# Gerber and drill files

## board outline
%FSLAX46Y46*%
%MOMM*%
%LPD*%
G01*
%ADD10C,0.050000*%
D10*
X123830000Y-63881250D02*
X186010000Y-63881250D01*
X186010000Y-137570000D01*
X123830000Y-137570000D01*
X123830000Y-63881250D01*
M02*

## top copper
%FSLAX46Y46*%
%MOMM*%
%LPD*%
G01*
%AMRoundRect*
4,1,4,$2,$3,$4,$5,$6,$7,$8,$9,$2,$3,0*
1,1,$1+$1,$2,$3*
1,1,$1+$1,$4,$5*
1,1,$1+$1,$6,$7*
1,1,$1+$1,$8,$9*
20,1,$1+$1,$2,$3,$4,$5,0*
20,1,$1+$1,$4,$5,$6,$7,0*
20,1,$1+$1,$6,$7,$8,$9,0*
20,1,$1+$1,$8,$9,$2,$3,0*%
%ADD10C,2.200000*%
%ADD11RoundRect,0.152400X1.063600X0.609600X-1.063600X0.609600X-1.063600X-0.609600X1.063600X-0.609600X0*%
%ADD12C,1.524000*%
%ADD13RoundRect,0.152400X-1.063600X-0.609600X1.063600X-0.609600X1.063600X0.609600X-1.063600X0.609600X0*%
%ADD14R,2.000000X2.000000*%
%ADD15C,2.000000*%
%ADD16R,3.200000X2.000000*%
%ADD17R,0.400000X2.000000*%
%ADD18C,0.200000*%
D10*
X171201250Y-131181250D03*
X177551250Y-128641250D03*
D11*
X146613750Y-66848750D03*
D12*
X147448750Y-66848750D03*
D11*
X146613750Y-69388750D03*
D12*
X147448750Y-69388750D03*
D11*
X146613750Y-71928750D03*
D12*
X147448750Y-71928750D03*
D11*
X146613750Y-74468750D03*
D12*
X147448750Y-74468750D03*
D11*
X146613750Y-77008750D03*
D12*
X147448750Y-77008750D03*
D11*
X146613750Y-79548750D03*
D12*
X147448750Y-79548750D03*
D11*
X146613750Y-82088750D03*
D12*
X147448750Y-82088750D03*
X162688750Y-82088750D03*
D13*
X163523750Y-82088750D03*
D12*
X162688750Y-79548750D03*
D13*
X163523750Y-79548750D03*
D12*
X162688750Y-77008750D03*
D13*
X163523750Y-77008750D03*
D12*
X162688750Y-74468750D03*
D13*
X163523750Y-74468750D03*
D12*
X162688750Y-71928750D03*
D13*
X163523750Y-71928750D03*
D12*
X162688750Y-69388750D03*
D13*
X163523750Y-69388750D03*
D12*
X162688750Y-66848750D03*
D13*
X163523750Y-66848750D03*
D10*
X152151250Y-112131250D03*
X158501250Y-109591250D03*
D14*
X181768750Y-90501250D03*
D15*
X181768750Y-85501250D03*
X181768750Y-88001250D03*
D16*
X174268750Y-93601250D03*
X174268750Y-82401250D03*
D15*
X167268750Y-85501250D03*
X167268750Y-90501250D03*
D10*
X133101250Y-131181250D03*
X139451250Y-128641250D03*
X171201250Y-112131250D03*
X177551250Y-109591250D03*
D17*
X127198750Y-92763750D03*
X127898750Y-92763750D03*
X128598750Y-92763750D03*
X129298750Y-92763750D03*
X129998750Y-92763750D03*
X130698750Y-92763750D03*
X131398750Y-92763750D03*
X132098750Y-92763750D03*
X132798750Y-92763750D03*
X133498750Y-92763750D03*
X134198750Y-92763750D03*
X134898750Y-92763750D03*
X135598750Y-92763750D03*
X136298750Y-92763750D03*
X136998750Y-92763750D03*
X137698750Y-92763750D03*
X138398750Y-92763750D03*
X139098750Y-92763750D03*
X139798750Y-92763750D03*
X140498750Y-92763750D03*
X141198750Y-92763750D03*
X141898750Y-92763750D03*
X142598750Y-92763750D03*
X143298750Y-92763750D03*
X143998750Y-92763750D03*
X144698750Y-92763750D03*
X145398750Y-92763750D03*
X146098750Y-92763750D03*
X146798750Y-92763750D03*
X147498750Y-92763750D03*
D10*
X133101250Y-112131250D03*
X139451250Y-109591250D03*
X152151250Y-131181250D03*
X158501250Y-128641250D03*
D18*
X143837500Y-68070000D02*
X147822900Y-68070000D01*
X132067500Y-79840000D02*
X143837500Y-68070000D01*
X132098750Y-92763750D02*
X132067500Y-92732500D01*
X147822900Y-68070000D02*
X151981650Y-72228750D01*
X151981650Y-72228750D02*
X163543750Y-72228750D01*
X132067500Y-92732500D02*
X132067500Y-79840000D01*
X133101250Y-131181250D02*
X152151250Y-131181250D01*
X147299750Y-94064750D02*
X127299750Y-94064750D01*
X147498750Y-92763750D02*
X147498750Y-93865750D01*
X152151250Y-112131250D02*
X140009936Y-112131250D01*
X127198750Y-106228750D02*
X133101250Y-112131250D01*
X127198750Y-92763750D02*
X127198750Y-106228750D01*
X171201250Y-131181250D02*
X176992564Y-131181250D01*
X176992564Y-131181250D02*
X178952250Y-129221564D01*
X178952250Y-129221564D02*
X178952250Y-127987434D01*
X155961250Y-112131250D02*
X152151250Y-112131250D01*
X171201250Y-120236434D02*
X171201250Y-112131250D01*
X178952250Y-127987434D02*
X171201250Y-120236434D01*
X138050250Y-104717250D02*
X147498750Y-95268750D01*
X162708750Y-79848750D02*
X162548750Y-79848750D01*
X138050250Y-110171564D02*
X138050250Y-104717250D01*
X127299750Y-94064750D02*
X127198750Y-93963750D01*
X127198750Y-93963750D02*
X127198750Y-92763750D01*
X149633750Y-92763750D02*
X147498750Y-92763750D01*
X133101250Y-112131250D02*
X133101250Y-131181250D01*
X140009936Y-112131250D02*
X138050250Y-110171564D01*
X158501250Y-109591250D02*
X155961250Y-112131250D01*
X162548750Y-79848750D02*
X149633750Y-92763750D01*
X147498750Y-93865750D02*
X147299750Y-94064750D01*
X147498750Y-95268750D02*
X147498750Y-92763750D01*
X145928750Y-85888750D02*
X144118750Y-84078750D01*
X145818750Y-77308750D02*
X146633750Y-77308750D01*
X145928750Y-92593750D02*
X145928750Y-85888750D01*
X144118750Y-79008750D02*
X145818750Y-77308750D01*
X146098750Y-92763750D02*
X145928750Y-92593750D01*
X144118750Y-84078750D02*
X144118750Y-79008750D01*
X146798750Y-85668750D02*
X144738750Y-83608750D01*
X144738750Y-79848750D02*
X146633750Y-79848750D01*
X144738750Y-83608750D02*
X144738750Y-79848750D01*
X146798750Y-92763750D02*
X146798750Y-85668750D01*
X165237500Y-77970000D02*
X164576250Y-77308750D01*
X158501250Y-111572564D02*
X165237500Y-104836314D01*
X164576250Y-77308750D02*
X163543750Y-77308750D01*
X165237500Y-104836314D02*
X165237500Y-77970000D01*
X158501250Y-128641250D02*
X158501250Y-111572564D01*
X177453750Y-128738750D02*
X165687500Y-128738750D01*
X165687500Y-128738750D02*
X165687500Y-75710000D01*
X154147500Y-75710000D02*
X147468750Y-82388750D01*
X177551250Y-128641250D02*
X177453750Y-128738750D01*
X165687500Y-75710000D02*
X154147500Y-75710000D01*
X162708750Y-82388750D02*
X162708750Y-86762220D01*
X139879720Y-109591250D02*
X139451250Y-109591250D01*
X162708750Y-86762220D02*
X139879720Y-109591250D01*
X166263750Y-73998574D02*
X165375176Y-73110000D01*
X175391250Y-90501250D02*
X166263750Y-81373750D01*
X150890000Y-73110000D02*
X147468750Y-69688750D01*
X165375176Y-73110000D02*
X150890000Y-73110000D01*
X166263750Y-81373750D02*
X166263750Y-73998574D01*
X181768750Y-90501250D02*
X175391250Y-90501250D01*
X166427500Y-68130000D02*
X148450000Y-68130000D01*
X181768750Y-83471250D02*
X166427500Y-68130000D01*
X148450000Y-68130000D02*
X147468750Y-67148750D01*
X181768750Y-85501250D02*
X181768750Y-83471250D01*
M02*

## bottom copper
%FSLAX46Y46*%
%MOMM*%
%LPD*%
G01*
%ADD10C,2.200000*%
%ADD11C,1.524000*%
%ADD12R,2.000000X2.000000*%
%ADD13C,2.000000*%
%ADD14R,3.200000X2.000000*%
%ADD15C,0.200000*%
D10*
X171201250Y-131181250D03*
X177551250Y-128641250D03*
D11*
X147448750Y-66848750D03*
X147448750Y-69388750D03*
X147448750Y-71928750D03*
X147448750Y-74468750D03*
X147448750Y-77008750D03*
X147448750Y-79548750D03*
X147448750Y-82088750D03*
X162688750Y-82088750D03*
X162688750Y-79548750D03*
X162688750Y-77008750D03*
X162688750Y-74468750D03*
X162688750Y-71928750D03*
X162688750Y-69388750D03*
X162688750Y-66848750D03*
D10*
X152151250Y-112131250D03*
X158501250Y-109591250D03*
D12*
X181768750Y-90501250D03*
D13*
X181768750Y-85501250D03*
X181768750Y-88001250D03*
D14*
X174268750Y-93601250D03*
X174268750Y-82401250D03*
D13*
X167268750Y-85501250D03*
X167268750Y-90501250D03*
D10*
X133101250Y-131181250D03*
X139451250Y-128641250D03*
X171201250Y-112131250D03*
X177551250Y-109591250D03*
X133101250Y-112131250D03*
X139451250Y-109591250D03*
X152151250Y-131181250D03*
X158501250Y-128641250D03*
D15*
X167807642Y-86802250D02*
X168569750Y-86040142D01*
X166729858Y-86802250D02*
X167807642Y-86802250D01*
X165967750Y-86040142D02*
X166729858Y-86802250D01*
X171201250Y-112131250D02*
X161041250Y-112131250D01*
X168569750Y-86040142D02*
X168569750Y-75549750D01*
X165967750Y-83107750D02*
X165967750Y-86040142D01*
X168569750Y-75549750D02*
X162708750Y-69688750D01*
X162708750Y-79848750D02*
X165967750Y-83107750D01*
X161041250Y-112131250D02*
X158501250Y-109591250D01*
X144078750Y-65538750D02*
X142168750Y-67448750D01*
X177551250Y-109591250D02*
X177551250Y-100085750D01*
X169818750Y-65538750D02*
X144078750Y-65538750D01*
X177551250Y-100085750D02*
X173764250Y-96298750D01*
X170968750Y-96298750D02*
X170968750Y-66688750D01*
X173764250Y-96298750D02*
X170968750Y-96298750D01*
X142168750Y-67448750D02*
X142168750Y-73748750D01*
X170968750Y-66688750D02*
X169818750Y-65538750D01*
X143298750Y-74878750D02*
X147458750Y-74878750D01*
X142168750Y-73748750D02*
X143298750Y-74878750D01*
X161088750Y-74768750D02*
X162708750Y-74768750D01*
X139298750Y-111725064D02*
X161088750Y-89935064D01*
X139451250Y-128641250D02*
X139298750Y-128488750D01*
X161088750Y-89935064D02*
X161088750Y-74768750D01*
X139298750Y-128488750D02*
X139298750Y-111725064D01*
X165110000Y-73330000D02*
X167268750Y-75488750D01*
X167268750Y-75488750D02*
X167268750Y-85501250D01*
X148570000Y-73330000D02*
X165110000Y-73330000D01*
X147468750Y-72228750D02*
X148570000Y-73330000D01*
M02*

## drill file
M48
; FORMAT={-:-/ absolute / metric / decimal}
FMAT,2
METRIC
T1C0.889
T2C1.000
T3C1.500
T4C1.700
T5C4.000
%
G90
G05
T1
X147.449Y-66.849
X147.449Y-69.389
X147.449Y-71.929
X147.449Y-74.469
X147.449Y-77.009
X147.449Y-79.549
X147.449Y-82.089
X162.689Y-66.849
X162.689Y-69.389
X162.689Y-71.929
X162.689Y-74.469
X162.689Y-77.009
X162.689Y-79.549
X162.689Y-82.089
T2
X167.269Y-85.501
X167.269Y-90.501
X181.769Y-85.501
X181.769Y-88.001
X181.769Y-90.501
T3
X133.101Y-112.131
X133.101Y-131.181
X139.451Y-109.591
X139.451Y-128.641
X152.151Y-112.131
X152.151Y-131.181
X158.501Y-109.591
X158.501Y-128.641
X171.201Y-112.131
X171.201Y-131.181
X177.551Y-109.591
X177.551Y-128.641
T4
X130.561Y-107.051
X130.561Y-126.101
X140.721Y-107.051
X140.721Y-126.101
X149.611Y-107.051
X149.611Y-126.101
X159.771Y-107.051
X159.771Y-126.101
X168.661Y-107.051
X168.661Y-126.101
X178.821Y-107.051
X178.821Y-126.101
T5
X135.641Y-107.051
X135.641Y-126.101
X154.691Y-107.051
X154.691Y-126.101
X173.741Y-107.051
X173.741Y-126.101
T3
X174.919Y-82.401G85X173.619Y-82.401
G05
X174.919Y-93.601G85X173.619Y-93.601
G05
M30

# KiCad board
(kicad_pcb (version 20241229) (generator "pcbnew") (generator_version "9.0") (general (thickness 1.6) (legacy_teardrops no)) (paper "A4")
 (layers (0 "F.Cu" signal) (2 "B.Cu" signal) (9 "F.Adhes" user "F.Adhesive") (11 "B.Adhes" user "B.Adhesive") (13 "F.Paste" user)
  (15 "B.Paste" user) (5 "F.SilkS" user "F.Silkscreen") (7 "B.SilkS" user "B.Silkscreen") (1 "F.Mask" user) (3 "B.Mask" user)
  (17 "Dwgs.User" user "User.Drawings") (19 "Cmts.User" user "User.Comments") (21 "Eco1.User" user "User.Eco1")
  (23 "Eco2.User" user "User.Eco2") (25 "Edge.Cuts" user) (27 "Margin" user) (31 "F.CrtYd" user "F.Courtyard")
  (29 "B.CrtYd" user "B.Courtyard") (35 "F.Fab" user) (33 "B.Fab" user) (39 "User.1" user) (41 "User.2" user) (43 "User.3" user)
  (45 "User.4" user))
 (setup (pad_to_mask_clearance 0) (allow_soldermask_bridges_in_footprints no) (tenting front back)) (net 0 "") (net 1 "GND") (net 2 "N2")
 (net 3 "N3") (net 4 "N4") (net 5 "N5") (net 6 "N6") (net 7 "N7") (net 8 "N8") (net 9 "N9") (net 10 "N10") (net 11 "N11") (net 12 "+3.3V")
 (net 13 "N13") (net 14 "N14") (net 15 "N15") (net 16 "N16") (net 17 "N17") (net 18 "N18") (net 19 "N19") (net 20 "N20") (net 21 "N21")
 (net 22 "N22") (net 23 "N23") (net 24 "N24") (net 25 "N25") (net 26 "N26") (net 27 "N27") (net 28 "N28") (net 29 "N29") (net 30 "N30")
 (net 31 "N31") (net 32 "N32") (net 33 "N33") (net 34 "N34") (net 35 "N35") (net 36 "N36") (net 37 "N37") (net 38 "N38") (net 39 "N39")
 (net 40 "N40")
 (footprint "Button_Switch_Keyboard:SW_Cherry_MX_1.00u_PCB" (layer "F.Cu") (at 171.20125 131.18125 180)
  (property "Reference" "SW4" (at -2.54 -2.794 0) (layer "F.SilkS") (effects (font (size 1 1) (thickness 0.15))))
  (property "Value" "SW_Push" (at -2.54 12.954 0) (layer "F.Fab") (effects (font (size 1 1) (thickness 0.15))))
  (pad "" np_thru_hole circle (at -7.62 5.08 180) (size 1.7 1.7) (drill 1.7) (layers "*.Cu" "*.Mask"))
  (pad "" np_thru_hole circle (at -2.54 5.08 180) (size 4 4) (drill 4) (layers "*.Cu" "*.Mask"))
  (pad "" np_thru_hole circle (at 2.54 5.08 180) (size 1.7 1.7) (drill 1.7) (layers "*.Cu" "*.Mask"))
  (pad "1" thru_hole circle (at 0 0 180) (size 2.2 2.2) (drill 1.5) (layers "*.Cu" "*.Mask") (remove_unused_layers no) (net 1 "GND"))
  (pad "2" thru_hole circle (at -6.35 2.54 180) (size 2.2 2.2) (drill 1.5) (layers "*.Cu" "*.Mask") (remove_unused_layers no) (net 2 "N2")))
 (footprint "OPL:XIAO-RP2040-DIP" (layer "F.Cu") (at 155.06875 74.46875)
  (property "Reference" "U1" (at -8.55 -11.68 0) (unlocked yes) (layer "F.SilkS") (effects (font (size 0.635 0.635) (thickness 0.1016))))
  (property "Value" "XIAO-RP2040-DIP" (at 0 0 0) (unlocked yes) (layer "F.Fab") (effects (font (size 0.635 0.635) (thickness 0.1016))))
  (pad "1" smd roundrect (at -8.455 -7.62 180) (size 2.432 1.524) (layers "F.Cu" "F.Mask") (roundrect_rratio 0.1) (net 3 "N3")
   (thermal_bridge_angle 45))
  (pad "1" thru_hole circle (at -7.62 -7.62 180) (size 1.524 1.524) (drill 0.889) (layers "*.Cu" "*.Mask") (remove_unused_layers no)
   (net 3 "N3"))
  (pad "2" smd roundrect (at -8.455 -5.08 180) (size 2.432 1.524) (layers "F.Cu" "F.Mask") (roundrect_rratio 0.1) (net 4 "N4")
   (thermal_bridge_angle 45))
  (pad "2" thru_hole circle (at -7.62 -5.08 180) (size 1.524 1.524) (drill 0.889) (layers "*.Cu" "*.Mask") (remove_unused_layers no)
   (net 4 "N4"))
  (pad "3" smd roundrect (at -8.455 -2.54 180) (size 2.432 1.524) (layers "F.Cu" "F.Mask") (roundrect_rratio 0.1) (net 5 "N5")
   (thermal_bridge_angle 45))
  (pad "3" thru_hole circle (at -7.62 -2.54 180) (size 1.524 1.524) (drill 0.889) (layers "*.Cu" "*.Mask") (remove_unused_layers no)
   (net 5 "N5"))
  (pad "4" smd roundrect (at -8.455 0 180) (size 2.432 1.524) (layers "F.Cu" "F.Mask") (roundrect_rratio 0.1) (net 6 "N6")
   (thermal_bridge_angle 45))
  (pad "4" thru_hole circle (at -7.62 0 180) (size 1.524 1.524) (drill 0.889) (layers "*.Cu" "*.Mask") (remove_unused_layers no)
   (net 6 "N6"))
  (pad "5" smd roundrect (at -8.455 2.54 180) (size 2.432 1.524) (layers "F.Cu" "F.Mask") (roundrect_rratio 0.1) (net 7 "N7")
   (thermal_bridge_angle 45))
  (pad "5" thru_hole circle (at -7.62 2.54 180) (size 1.524 1.524) (drill 0.889) (layers "*.Cu" "*.Mask") (remove_unused_layers no)
   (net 7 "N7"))
  (pad "6" smd roundrect (at -8.455 5.08 180) (size 2.432 1.524) (layers "F.Cu" "F.Mask") (roundrect_rratio 0.1) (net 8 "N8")
   (thermal_bridge_angle 45))
  (pad "6" thru_hole circle (at -7.62 5.08 180) (size 1.524 1.524) (drill 0.889) (layers "*.Cu" "*.Mask") (remove_unused_layers no)
   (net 8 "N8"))
  (pad "7" smd roundrect (at -8.455 7.62 180) (size 2.432 1.524) (layers "F.Cu" "F.Mask") (roundrect_rratio 0.1) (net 2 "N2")
   (thermal_bridge_angle 45))
  (pad "7" thru_hole circle (at -7.62 7.62 180) (size 1.524 1.524) (drill 0.889) (layers "*.Cu" "*.Mask") (remove_unused_layers no)
   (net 2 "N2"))
  (pad "8" thru_hole circle (at 7.62 7.62) (size 1.524 1.524) (drill 0.889) (layers "*.Cu" "*.Mask") (remove_unused_layers no) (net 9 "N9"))
  (pad "8" smd roundrect (at 8.455 7.62) (size 2.432 1.524) (layers "F.Cu" "F.Mask") (roundrect_rratio 0.1) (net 9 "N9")
   (thermal_bridge_angle 45))
  (pad "9" thru_hole circle (at 7.62 5.08) (size 1.524 1.524) (drill 0.889) (layers "*.Cu" "*.Mask") (remove_unused_layers no) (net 1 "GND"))
  (pad "9" smd roundrect (at 8.455 5.08) (size 2.432 1.524) (layers "F.Cu" "F.Mask") (roundrect_rratio 0.1) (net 1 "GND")
   (thermal_bridge_angle 45))
  (pad "10" thru_hole circle (at 7.62 2.54) (size 1.524 1.524) (drill 0.889) (layers "*.Cu" "*.Mask") (remove_unused_layers no)
   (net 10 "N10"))
  (pad "10" smd roundrect (at 8.455 2.54) (size 2.432 1.524) (layers "F.Cu" "F.Mask") (roundrect_rratio 0.1) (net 10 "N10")
   (thermal_bridge_angle 45))
  (pad "11" thru_hole circle (at 7.62 0) (size 1.524 1.524) (drill 0.889) (layers "*.Cu" "*.Mask") (remove_unused_layers no) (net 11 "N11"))
  (pad "11" smd roundrect (at 8.455 0) (size 2.432 1.524) (layers "F.Cu" "F.Mask") (roundrect_rratio 0.1) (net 11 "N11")
   (thermal_bridge_angle 45))
  (pad "12" thru_hole circle (at 7.62 -2.54) (size 1.524 1.524) (drill 0.889) (layers "*.Cu" "*.Mask") (remove_unused_layers no)
   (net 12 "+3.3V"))
  (pad "12" smd roundrect (at 8.455 -2.54) (size 2.432 1.524) (layers "F.Cu" "F.Mask") (roundrect_rratio 0.1) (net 12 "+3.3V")
   (thermal_bridge_angle 45))
  (pad "13" thru_hole circle (at 7.62 -5.08) (size 1.524 1.524) (drill 0.889) (layers "*.Cu" "*.Mask") (remove_unused_layers no)
   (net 1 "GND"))
  (pad "13" smd roundrect (at 8.455 -5.08) (size 2.432 1.524) (layers "F.Cu" "F.Mask") (roundrect_rratio 0.1) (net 1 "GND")
   (thermal_bridge_angle 45))
  (pad "14" thru_hole circle (at 7.62 -7.62) (size 1.524 1.524) (drill 0.889) (layers "*.Cu" "*.Mask") (remove_unused_layers no)
   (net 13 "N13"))
  (pad "14" smd roundrect (at 8.455 -7.62) (size 2.432 1.524) (layers "F.Cu" "F.Mask") (roundrect_rratio 0.1) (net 13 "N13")
   (thermal_bridge_angle 45)))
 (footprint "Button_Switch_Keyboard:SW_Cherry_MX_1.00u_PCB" (layer "F.Cu") (at 152.15125 112.13125 180)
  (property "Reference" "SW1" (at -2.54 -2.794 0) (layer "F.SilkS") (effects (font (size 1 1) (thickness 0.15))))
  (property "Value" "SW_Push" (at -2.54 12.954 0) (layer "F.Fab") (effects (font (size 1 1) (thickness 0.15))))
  (pad "" np_thru_hole circle (at -7.62 5.08 180) (size 1.7 1.7) (drill 1.7) (layers "*.Cu" "*.Mask"))
  (pad "" np_thru_hole circle (at -2.54 5.08 180) (size 4 4) (drill 4) (layers "*.Cu" "*.Mask"))
  (pad "" np_thru_hole circle (at 2.54 5.08 180) (size 1.7 1.7) (drill 1.7) (layers "*.Cu" "*.Mask"))
  (pad "1" thru_hole circle (at 0 0 180) (size 2.2 2.2) (drill 1.5) (layers "*.Cu" "*.Mask") (remove_unused_layers no) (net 1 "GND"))
  (pad "2" thru_hole circle (at -6.35 2.54 180) (size 2.2 2.2) (drill 1.5) (layers "*.Cu" "*.Mask") (remove_unused_layers no) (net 1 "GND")))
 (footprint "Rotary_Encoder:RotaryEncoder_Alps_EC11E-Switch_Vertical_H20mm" (layer "F.Cu") (at 181.76875 90.50125 180)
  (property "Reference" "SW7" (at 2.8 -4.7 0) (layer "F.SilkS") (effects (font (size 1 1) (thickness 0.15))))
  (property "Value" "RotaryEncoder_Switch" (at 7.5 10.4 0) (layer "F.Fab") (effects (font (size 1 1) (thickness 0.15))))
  (pad "A" thru_hole rect (at 0 0 180) (size 2 2) (drill 1) (layers "*.Cu" "*.Mask") (remove_unused_layers no) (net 4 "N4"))
  (pad "B" thru_hole circle (at 0 5 180) (size 2 2) (drill 1) (layers "*.Cu" "*.Mask") (remove_unused_layers no) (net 3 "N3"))
  (pad "C" thru_hole circle (at 0 2.5 180) (size 2 2) (drill 1) (layers "*.Cu" "*.Mask") (remove_unused_layers no) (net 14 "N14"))
  (pad "MP" thru_hole rect (at 7.5 -3.1 180) (size 3.2 2) (drill oval 2.8 1.5) (layers "*.Cu" "*.Mask") (remove_unused_layers no))
  (pad "MP" thru_hole rect (at 7.5 8.1 180) (size 3.2 2) (drill oval 2.8 1.5) (layers "*.Cu" "*.Mask") (remove_unused_layers no))
  (pad "S1" thru_hole circle (at 14.5 5 180) (size 2 2) (drill 1) (layers "*.Cu" "*.Mask") (remove_unused_layers no) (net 5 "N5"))
  (pad "S2" thru_hole circle (at 14.5 0 180) (size 2 2) (drill 1) (layers "*.Cu" "*.Mask") (remove_unused_layers no) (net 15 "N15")))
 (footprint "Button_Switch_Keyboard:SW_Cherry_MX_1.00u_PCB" (layer "F.Cu") (at 133.10125 131.18125 180)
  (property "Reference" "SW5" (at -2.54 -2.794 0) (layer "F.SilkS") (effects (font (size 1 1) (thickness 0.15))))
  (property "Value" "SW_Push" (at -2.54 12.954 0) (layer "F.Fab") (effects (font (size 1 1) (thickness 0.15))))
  (pad "" np_thru_hole circle (at -7.62 5.08 180) (size 1.7 1.7) (drill 1.7) (layers "*.Cu" "*.Mask"))
  (pad "" np_thru_hole circle (at -2.54 5.08 180) (size 4 4) (drill 4) (layers "*.Cu" "*.Mask"))
  (pad "" np_thru_hole circle (at 2.54 5.08 180) (size 1.7 1.7) (drill 1.7) (layers "*.Cu" "*.Mask"))
  (pad "1" thru_hole circle (at 0 0 180) (size 2.2 2.2) (drill 1.5) (layers "*.Cu" "*.Mask") (remove_unused_layers no) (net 1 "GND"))
  (pad "2" thru_hole circle (at -6.35 2.54 180) (size 2.2 2.2) (drill 1.5) (layers "*.Cu" "*.Mask") (remove_unused_layers no) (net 11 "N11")))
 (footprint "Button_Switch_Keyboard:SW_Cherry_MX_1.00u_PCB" (layer "F.Cu") (at 171.20125 112.13125 180)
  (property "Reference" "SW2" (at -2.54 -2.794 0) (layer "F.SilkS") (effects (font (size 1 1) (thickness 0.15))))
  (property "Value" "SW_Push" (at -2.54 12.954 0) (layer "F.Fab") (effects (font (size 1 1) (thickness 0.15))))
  (pad "" np_thru_hole circle (at -7.62 5.08 180) (size 1.7 1.7) (drill 1.7) (layers "*.Cu" "*.Mask"))
  (pad "" np_thru_hole circle (at -2.54 5.08 180) (size 4 4) (drill 4) (layers "*.Cu" "*.Mask"))
  (pad "" np_thru_hole circle (at 2.54 5.08 180) (size 1.7 1.7) (drill 1.7) (layers "*.Cu" "*.Mask"))
  (pad "1" thru_hole circle (at 0 0 180) (size 2.2 2.2) (drill 1.5) (layers "*.Cu" "*.Mask") (remove_unused_layers no) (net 1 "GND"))
  (pad "2" thru_hole circle (at -6.35 2.54 180) (size 2.2 2.2) (drill 1.5) (layers "*.Cu" "*.Mask") (remove_unused_layers no) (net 6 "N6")))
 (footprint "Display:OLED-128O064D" (layer "F.Cu") (at 137.34875 92.76375)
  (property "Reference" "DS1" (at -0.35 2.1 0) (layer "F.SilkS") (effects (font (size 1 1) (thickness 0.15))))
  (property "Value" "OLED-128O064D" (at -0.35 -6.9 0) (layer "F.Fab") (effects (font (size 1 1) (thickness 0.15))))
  (pad "1" smd rect (at -10.15 0) (size 0.4 2) (layers "F.Cu" "F.Mask" "F.Paste") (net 1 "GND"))
  (pad "2" smd rect (at -9.45 0) (size 0.4 2) (layers "F.Cu" "F.Mask" "F.Paste") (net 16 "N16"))
  (pad "3" smd rect (at -8.75 0) (size 0.4 2) (layers "F.Cu" "F.Mask" "F.Paste") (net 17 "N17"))
  (pad "4" smd rect (at -8.05 0) (size 0.4 2) (layers "F.Cu" "F.Mask" "F.Paste") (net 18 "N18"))
  (pad "5" smd rect (at -7.35 0) (size 0.4 2) (layers "F.Cu" "F.Mask" "F.Paste") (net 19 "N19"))
  (pad "6" smd rect (at -6.65 0) (size 0.4 2) (layers "F.Cu" "F.Mask" "F.Paste") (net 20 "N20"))
  (pad "7" smd rect (at -5.95 0) (size 0.4 2) (layers "F.Cu" "F.Mask" "F.Paste") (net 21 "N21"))
  (pad "8" smd rect (at -5.25 0) (size 0.4 2) (layers "F.Cu" "F.Mask" "F.Paste") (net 12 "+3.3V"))
  (pad "9" smd rect (at -4.55 0) (size 0.4 2) (layers "F.Cu" "F.Mask" "F.Paste") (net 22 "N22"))
  (pad "10" smd rect (at -3.85 0) (size 0.4 2) (layers "F.Cu" "F.Mask" "F.Paste") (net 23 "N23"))
  (pad "11" smd rect (at -3.15 0) (size 0.4 2) (layers "F.Cu" "F.Mask" "F.Paste") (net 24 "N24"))
  (pad "12" smd rect (at -2.45 0) (size 0.4 2) (layers "F.Cu" "F.Mask" "F.Paste") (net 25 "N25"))
  (pad "13" smd rect (at -1.75 0) (size 0.4 2) (layers "F.Cu" "F.Mask" "F.Paste") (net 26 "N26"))
  (pad "14" smd rect (at -1.05 0) (size 0.4 2) (layers "F.Cu" "F.Mask" "F.Paste") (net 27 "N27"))
  (pad "15" smd rect (at -0.35 0) (size 0.4 2) (layers "F.Cu" "F.Mask" "F.Paste") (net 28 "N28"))
  (pad "16" smd rect (at 0.35 0) (size 0.4 2) (layers "F.Cu" "F.Mask" "F.Paste") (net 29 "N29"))
  (pad "17" smd rect (at 1.05 0) (size 0.4 2) (layers "F.Cu" "F.Mask" "F.Paste") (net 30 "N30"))
  (pad "18" smd rect (at 1.75 0) (size 0.4 2) (layers "F.Cu" "F.Mask" "F.Paste") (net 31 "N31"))
  (pad "19" smd rect (at 2.45 0) (size 0.4 2) (layers "F.Cu" "F.Mask" "F.Paste") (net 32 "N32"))
  (pad "20" smd rect (at 3.15 0) (size 0.4 2) (layers "F.Cu" "F.Mask" "F.Paste") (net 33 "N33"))
  (pad "21" smd rect (at 3.85 0) (size 0.4 2) (layers "F.Cu" "F.Mask" "F.Paste") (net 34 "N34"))
  (pad "22" smd rect (at 4.55 0) (size 0.4 2) (layers "F.Cu" "F.Mask" "F.Paste") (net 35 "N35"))
  (pad "23" smd rect (at 5.25 0) (size 0.4 2) (layers "F.Cu" "F.Mask" "F.Paste") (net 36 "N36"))
  (pad "24" smd rect (at 5.95 0) (size 0.4 2) (layers "F.Cu" "F.Mask" "F.Paste") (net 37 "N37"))
  (pad "25" smd rect (at 6.65 0) (size 0.4 2) (layers "F.Cu" "F.Mask" "F.Paste") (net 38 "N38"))
  (pad "26" smd rect (at 7.35 0) (size 0.4 2) (layers "F.Cu" "F.Mask" "F.Paste") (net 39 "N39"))
  (pad "27" smd rect (at 8.05 0) (size 0.4 2) (layers "F.Cu" "F.Mask" "F.Paste") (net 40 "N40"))
  (pad "28" smd rect (at 8.75 0) (size 0.4 2) (layers "F.Cu" "F.Mask" "F.Paste") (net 7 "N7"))
  (pad "29" smd rect (at 9.45 0) (size 0.4 2) (layers "F.Cu" "F.Mask" "F.Paste") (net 8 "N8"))
  (pad "30" smd rect (at 10.15 0) (size 0.4 2) (layers "F.Cu" "F.Mask" "F.Paste") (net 1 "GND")))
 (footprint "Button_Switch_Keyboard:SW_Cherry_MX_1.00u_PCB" (layer "F.Cu") (at 133.10125 112.13125 180)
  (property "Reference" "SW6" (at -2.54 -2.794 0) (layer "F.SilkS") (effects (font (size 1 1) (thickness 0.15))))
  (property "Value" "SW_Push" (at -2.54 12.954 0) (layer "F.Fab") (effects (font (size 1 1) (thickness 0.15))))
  (pad "" np_thru_hole circle (at -7.62 5.08 180) (size 1.7 1.7) (drill 1.7) (layers "*.Cu" "*.Mask"))
  (pad "" np_thru_hole circle (at -2.54 5.08 180) (size 4 4) (drill 4) (layers "*.Cu" "*.Mask"))
  (pad "" np_thru_hole circle (at 2.54 5.08 180) (size 1.7 1.7) (drill 1.7) (layers "*.Cu" "*.Mask"))
  (pad "1" thru_hole circle (at 0 0 180) (size 2.2 2.2) (drill 1.5) (layers "*.Cu" "*.Mask") (remove_unused_layers no) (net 1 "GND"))
  (pad "2" thru_hole circle (at -6.35 2.54 180) (size 2.2 2.2) (drill 1.5) (layers "*.Cu" "*.Mask") (remove_unused_layers no) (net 9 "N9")))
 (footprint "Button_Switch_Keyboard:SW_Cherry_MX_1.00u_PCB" (layer "F.Cu") (at 152.15125 131.18125 180)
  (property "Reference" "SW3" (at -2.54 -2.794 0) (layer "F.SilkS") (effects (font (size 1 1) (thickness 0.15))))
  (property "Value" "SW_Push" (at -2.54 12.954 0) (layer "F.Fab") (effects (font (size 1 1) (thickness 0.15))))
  (pad "" np_thru_hole circle (at -7.62 5.08 180) (size 1.7 1.7) (drill 1.7) (layers "*.Cu" "*.Mask"))
  (pad "" np_thru_hole circle (at -2.54 5.08 180) (size 4 4) (drill 4) (layers "*.Cu" "*.Mask"))
  (pad "" np_thru_hole circle (at 2.54 5.08 180) (size 1.7 1.7) (drill 1.7) (layers "*.Cu" "*.Mask"))
  (pad "1" thru_hole circle (at 0 0 180) (size 2.2 2.2) (drill 1.5) (layers "*.Cu" "*.Mask") (remove_unused_layers no) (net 1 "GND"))
  (pad "2" thru_hole circle (at -6.35 2.54 180) (size 2.2 2.2) (drill 1.5) (layers "*.Cu" "*.Mask") (remove_unused_layers no) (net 10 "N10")))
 (gr_rect (start 123.83 63.88125) (end 186.01 137.57) (stroke (width 0.05) (type default)) (fill no) (layer "Edge.Cuts"))
 (segment (start 143.8375 68.07) (end 147.8229 68.07) (width 0.2) (layer "F.Cu") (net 12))
 (segment (start 132.0675 79.84) (end 143.8375 68.07) (width 0.2) (layer "F.Cu") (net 12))
 (segment (start 132.09875 92.76375) (end 132.0675 92.7325) (width 0.2) (layer "F.Cu") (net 12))
 (segment (start 147.8229 68.07) (end 151.98165 72.22875) (width 0.2) (layer "F.Cu") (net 12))
 (segment (start 151.98165 72.22875) (end 163.54375 72.22875) (width 0.2) (layer "F.Cu") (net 12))
 (segment (start 132.0675 92.7325) (end 132.0675 79.84) (width 0.2) (layer "F.Cu") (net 12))
 (segment (start 133.10125 131.18125) (end 152.15125 131.18125) (width 0.2) (layer "F.Cu") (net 1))
 (segment (start 147.29975 94.06475) (end 127.29975 94.06475) (width 0.2) (layer "F.Cu") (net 1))
 (segment (start 147.49875 92.76375) (end 147.49875 93.86575) (width 0.2) (layer "F.Cu") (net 1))
 (segment (start 152.15125 112.13125) (end 140.009936 112.13125) (width 0.2) (layer "F.Cu") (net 1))
 (segment (start 127.19875 106.22875) (end 133.10125 112.13125) (width 0.2) (layer "F.Cu") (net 1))
 (segment (start 127.19875 92.76375) (end 127.19875 106.22875) (width 0.2) (layer "F.Cu") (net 1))
 (segment (start 171.20125 131.18125) (end 176.992564 131.18125) (width 0.2) (layer "F.Cu") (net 1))
 (segment (start 176.992564 131.18125) (end 178.95225 129.221564) (width 0.2) (layer "F.Cu") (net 1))
 (segment (start 178.95225 129.221564) (end 178.95225 127.987434) (width 0.2) (layer "F.Cu") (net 1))
 (segment (start 155.96125 112.13125) (end 152.15125 112.13125) (width 0.2) (layer "F.Cu") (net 1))
 (segment (start 171.20125 120.236434) (end 171.20125 112.13125) (width 0.2) (layer "F.Cu") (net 1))
 (segment (start 178.95225 127.987434) (end 171.20125 120.236434) (width 0.2) (layer "F.Cu") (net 1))
 (segment (start 138.05025 104.71725) (end 147.49875 95.26875) (width 0.2) (layer "F.Cu") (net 1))
 (segment (start 162.70875 79.84875) (end 162.54875 79.84875) (width 0.2) (layer "F.Cu") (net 1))
 (segment (start 138.05025 110.171564) (end 138.05025 104.71725) (width 0.2) (layer "F.Cu") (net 1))
 (segment (start 127.29975 94.06475) (end 127.19875 93.96375) (width 0.2) (layer "F.Cu") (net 1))
 (segment (start 127.19875 93.96375) (end 127.19875 92.76375) (width 0.2) (layer "F.Cu") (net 1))
 (segment (start 149.63375 92.76375) (end 147.49875 92.76375) (width 0.2) (layer "F.Cu") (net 1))
 (segment (start 133.10125 112.13125) (end 133.10125 131.18125) (width 0.2) (layer "F.Cu") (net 1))
 (segment (start 140.009936 112.13125) (end 138.05025 110.171564) (width 0.2) (layer "F.Cu") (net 1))
 (segment (start 158.50125 109.59125) (end 155.96125 112.13125) (width 0.2) (layer "F.Cu") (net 1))
 (segment (start 162.54875 79.84875) (end 149.63375 92.76375) (width 0.2) (layer "F.Cu") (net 1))
 (segment (start 147.49875 93.86575) (end 147.29975 94.06475) (width 0.2) (layer "F.Cu") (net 1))
 (segment (start 147.49875 95.26875) (end 147.49875 92.76375) (width 0.2) (layer "F.Cu") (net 1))
 (segment (start 167.807642 86.80225) (end 168.56975 86.040142) (width 0.2) (layer "B.Cu") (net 1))
 (segment (start 166.729858 86.80225) (end 167.807642 86.80225) (width 0.2) (layer "B.Cu") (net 1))
 (segment (start 165.96775 86.040142) (end 166.729858 86.80225) (width 0.2) (layer "B.Cu") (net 1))
 (segment (start 171.20125 112.13125) (end 161.04125 112.13125) (width 0.2) (layer "B.Cu") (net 1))
 (segment (start 168.56975 86.040142) (end 168.56975 75.54975) (width 0.2) (layer "B.Cu") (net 1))
 (segment (start 165.96775 83.10775) (end 165.96775 86.040142) (width 0.2) (layer "B.Cu") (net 1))
 (segment (start 168.56975 75.54975) (end 162.70875 69.68875) (width 0.2) (layer "B.Cu") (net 1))
 (segment (start 162.70875 79.84875) (end 165.96775 83.10775) (width 0.2) (layer "B.Cu") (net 1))
 (segment (start 161.04125 112.13125) (end 158.50125 109.59125) (width 0.2) (layer "B.Cu") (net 1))
 (segment (start 145.92875 85.88875) (end 144.11875 84.07875) (width 0.2) (layer "F.Cu") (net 7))
 (segment (start 145.81875 77.30875) (end 146.63375 77.30875) (width 0.2) (layer "F.Cu") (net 7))
 (segment (start 145.92875 92.59375) (end 145.92875 85.88875) (width 0.2) (layer "F.Cu") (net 7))
 (segment (start 144.11875 79.00875) (end 145.81875 77.30875) (width 0.2) (layer "F.Cu") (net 7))
 (segment (start 146.09875 92.76375) (end 145.92875 92.59375) (width 0.2) (layer "F.Cu") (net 7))
 (segment (start 144.11875 84.07875) (end 144.11875 79.00875) (width 0.2) (layer "F.Cu") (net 7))
 (segment (start 146.79875 85.66875) (end 144.73875 83.60875) (width 0.2) (layer "F.Cu") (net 8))
 (segment (start 144.73875 79.84875) (end 146.63375 79.84875) (width 0.2) (layer "F.Cu") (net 8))
 (segment (start 144.73875 83.60875) (end 144.73875 79.84875) (width 0.2) (layer "F.Cu") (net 8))
 (segment (start 146.79875 92.76375) (end 146.79875 85.66875) (width 0.2) (layer "F.Cu") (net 8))
 (segment (start 144.07875 65.53875) (end 142.16875 67.44875) (width 0.2) (layer "B.Cu") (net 6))
 (segment (start 177.55125 109.59125) (end 177.55125 100.08575) (width 0.2) (layer "B.Cu") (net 6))
 (segment (start 169.81875 65.53875) (end 144.07875 65.53875) (width 0.2) (layer "B.Cu") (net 6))
 (segment (start 177.55125 100.08575) (end 173.76425 96.29875) (width 0.2) (layer "B.Cu") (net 6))
 (segment (start 170.96875 96.29875) (end 170.96875 66.68875) (width 0.2) (layer "B.Cu") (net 6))
 (segment (start 173.76425 96.29875) (end 170.96875 96.29875) (width 0.2) (layer "B.Cu") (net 6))
 (segment (start 142.16875 67.44875) (end 142.16875 73.74875) (width 0.2) (layer "B.Cu") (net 6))
 (segment (start 170.96875 66.68875) (end 169.81875 65.53875) (width 0.2) (layer "B.Cu") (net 6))
 (segment (start 143.29875 74.87875) (end 147.45875 74.87875) (width 0.2) (layer "B.Cu") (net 6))
 (segment (start 142.16875 73.74875) (end 143.29875 74.87875) (width 0.2) (layer "B.Cu") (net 6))
 (segment (start 165.2375 77.97) (end 164.57625 77.30875) (width 0.2) (layer "F.Cu") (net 10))
 (segment (start 158.50125 111.572564) (end 165.2375 104.836314) (width 0.2) (layer "F.Cu") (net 10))
 (segment (start 164.57625 77.30875) (end 163.54375 77.30875) (width 0.2) (layer "F.Cu") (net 10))
 (segment (start 165.2375 104.836314) (end 165.2375 77.97) (width 0.2) (layer "F.Cu") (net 10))
 (segment (start 158.50125 128.64125) (end 158.50125 111.572564) (width 0.2) (layer "F.Cu") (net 10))
 (segment (start 177.45375 128.73875) (end 165.6875 128.73875) (width 0.2) (layer "F.Cu") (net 2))
 (segment (start 165.6875 128.73875) (end 165.6875 75.71) (width 0.2) (layer "F.Cu") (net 2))
 (segment (start 154.1475 75.71) (end 147.46875 82.38875) (width 0.2) (layer "F.Cu") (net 2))
 (segment (start 177.55125 128.64125) (end 177.45375 128.73875) (width 0.2) (layer "F.Cu") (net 2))
 (segment (start 165.6875 75.71) (end 154.1475 75.71) (width 0.2) (layer "F.Cu") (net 2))
 (segment (start 161.08875 74.76875) (end 162.70875 74.76875) (width 0.2) (layer "B.Cu") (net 11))
 (segment (start 139.29875 111.725064) (end 161.08875 89.935064) (width 0.2) (layer "B.Cu") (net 11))
 (segment (start 139.45125 128.64125) (end 139.29875 128.48875) (width 0.2) (layer "B.Cu") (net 11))
 (segment (start 161.08875 89.935064) (end 161.08875 74.76875) (width 0.2) (layer "B.Cu") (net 11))
 (segment (start 139.29875 128.48875) (end 139.29875 111.725064) (width 0.2) (layer "B.Cu") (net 11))
 (segment (start 162.70875 82.38875) (end 162.70875 86.76222) (width 0.2) (layer "F.Cu") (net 9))
 (segment (start 139.87972 109.59125) (end 139.45125 109.59125) (width 0.2) (layer "F.Cu") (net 9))
 (segment (start 162.70875 86.76222) (end 139.87972 109.59125) (width 0.2) (layer "F.Cu") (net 9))
 (segment (start 165.11 73.33) (end 167.26875 75.48875) (width 0.2) (layer "B.Cu") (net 5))
 (segment (start 167.26875 75.48875) (end 167.26875 85.50125) (width 0.2) (layer "B.Cu") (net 5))
 (segment (start 148.57 73.33) (end 165.11 73.33) (width 0.2) (layer "B.Cu") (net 5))
 (segment (start 147.46875 72.22875) (end 148.57 73.33) (width 0.2) (layer "B.Cu") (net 5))
 (segment (start 166.26375 73.998574) (end 165.375176 73.11) (width 0.2) (layer "F.Cu") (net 4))
 (segment (start 175.39125 90.50125) (end 166.26375 81.37375) (width 0.2) (layer "F.Cu") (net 4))
 (segment (start 150.89 73.11) (end 147.46875 69.68875) (width 0.2) (layer "F.Cu") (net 4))
 (segment (start 165.375176 73.11) (end 150.89 73.11) (width 0.2) (layer "F.Cu") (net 4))
 (segment (start 166.26375 81.37375) (end 166.26375 73.998574) (width 0.2) (layer "F.Cu") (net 4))
 (segment (start 181.76875 90.50125) (end 175.39125 90.50125) (width 0.2) (layer "F.Cu") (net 4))
 (segment (start 166.4275 68.13) (end 148.45 68.13) (width 0.2) (layer "F.Cu") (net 3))
 (segment (start 181.76875 83.47125) (end 166.4275 68.13) (width 0.2) (layer "F.Cu") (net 3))
 (segment (start 148.45 68.13) (end 147.46875 67.14875) (width 0.2) (layer "F.Cu") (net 3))
 (segment (start 181.76875 85.50125) (end 181.76875 83.47125) (width 0.2) (layer "F.Cu") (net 3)))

